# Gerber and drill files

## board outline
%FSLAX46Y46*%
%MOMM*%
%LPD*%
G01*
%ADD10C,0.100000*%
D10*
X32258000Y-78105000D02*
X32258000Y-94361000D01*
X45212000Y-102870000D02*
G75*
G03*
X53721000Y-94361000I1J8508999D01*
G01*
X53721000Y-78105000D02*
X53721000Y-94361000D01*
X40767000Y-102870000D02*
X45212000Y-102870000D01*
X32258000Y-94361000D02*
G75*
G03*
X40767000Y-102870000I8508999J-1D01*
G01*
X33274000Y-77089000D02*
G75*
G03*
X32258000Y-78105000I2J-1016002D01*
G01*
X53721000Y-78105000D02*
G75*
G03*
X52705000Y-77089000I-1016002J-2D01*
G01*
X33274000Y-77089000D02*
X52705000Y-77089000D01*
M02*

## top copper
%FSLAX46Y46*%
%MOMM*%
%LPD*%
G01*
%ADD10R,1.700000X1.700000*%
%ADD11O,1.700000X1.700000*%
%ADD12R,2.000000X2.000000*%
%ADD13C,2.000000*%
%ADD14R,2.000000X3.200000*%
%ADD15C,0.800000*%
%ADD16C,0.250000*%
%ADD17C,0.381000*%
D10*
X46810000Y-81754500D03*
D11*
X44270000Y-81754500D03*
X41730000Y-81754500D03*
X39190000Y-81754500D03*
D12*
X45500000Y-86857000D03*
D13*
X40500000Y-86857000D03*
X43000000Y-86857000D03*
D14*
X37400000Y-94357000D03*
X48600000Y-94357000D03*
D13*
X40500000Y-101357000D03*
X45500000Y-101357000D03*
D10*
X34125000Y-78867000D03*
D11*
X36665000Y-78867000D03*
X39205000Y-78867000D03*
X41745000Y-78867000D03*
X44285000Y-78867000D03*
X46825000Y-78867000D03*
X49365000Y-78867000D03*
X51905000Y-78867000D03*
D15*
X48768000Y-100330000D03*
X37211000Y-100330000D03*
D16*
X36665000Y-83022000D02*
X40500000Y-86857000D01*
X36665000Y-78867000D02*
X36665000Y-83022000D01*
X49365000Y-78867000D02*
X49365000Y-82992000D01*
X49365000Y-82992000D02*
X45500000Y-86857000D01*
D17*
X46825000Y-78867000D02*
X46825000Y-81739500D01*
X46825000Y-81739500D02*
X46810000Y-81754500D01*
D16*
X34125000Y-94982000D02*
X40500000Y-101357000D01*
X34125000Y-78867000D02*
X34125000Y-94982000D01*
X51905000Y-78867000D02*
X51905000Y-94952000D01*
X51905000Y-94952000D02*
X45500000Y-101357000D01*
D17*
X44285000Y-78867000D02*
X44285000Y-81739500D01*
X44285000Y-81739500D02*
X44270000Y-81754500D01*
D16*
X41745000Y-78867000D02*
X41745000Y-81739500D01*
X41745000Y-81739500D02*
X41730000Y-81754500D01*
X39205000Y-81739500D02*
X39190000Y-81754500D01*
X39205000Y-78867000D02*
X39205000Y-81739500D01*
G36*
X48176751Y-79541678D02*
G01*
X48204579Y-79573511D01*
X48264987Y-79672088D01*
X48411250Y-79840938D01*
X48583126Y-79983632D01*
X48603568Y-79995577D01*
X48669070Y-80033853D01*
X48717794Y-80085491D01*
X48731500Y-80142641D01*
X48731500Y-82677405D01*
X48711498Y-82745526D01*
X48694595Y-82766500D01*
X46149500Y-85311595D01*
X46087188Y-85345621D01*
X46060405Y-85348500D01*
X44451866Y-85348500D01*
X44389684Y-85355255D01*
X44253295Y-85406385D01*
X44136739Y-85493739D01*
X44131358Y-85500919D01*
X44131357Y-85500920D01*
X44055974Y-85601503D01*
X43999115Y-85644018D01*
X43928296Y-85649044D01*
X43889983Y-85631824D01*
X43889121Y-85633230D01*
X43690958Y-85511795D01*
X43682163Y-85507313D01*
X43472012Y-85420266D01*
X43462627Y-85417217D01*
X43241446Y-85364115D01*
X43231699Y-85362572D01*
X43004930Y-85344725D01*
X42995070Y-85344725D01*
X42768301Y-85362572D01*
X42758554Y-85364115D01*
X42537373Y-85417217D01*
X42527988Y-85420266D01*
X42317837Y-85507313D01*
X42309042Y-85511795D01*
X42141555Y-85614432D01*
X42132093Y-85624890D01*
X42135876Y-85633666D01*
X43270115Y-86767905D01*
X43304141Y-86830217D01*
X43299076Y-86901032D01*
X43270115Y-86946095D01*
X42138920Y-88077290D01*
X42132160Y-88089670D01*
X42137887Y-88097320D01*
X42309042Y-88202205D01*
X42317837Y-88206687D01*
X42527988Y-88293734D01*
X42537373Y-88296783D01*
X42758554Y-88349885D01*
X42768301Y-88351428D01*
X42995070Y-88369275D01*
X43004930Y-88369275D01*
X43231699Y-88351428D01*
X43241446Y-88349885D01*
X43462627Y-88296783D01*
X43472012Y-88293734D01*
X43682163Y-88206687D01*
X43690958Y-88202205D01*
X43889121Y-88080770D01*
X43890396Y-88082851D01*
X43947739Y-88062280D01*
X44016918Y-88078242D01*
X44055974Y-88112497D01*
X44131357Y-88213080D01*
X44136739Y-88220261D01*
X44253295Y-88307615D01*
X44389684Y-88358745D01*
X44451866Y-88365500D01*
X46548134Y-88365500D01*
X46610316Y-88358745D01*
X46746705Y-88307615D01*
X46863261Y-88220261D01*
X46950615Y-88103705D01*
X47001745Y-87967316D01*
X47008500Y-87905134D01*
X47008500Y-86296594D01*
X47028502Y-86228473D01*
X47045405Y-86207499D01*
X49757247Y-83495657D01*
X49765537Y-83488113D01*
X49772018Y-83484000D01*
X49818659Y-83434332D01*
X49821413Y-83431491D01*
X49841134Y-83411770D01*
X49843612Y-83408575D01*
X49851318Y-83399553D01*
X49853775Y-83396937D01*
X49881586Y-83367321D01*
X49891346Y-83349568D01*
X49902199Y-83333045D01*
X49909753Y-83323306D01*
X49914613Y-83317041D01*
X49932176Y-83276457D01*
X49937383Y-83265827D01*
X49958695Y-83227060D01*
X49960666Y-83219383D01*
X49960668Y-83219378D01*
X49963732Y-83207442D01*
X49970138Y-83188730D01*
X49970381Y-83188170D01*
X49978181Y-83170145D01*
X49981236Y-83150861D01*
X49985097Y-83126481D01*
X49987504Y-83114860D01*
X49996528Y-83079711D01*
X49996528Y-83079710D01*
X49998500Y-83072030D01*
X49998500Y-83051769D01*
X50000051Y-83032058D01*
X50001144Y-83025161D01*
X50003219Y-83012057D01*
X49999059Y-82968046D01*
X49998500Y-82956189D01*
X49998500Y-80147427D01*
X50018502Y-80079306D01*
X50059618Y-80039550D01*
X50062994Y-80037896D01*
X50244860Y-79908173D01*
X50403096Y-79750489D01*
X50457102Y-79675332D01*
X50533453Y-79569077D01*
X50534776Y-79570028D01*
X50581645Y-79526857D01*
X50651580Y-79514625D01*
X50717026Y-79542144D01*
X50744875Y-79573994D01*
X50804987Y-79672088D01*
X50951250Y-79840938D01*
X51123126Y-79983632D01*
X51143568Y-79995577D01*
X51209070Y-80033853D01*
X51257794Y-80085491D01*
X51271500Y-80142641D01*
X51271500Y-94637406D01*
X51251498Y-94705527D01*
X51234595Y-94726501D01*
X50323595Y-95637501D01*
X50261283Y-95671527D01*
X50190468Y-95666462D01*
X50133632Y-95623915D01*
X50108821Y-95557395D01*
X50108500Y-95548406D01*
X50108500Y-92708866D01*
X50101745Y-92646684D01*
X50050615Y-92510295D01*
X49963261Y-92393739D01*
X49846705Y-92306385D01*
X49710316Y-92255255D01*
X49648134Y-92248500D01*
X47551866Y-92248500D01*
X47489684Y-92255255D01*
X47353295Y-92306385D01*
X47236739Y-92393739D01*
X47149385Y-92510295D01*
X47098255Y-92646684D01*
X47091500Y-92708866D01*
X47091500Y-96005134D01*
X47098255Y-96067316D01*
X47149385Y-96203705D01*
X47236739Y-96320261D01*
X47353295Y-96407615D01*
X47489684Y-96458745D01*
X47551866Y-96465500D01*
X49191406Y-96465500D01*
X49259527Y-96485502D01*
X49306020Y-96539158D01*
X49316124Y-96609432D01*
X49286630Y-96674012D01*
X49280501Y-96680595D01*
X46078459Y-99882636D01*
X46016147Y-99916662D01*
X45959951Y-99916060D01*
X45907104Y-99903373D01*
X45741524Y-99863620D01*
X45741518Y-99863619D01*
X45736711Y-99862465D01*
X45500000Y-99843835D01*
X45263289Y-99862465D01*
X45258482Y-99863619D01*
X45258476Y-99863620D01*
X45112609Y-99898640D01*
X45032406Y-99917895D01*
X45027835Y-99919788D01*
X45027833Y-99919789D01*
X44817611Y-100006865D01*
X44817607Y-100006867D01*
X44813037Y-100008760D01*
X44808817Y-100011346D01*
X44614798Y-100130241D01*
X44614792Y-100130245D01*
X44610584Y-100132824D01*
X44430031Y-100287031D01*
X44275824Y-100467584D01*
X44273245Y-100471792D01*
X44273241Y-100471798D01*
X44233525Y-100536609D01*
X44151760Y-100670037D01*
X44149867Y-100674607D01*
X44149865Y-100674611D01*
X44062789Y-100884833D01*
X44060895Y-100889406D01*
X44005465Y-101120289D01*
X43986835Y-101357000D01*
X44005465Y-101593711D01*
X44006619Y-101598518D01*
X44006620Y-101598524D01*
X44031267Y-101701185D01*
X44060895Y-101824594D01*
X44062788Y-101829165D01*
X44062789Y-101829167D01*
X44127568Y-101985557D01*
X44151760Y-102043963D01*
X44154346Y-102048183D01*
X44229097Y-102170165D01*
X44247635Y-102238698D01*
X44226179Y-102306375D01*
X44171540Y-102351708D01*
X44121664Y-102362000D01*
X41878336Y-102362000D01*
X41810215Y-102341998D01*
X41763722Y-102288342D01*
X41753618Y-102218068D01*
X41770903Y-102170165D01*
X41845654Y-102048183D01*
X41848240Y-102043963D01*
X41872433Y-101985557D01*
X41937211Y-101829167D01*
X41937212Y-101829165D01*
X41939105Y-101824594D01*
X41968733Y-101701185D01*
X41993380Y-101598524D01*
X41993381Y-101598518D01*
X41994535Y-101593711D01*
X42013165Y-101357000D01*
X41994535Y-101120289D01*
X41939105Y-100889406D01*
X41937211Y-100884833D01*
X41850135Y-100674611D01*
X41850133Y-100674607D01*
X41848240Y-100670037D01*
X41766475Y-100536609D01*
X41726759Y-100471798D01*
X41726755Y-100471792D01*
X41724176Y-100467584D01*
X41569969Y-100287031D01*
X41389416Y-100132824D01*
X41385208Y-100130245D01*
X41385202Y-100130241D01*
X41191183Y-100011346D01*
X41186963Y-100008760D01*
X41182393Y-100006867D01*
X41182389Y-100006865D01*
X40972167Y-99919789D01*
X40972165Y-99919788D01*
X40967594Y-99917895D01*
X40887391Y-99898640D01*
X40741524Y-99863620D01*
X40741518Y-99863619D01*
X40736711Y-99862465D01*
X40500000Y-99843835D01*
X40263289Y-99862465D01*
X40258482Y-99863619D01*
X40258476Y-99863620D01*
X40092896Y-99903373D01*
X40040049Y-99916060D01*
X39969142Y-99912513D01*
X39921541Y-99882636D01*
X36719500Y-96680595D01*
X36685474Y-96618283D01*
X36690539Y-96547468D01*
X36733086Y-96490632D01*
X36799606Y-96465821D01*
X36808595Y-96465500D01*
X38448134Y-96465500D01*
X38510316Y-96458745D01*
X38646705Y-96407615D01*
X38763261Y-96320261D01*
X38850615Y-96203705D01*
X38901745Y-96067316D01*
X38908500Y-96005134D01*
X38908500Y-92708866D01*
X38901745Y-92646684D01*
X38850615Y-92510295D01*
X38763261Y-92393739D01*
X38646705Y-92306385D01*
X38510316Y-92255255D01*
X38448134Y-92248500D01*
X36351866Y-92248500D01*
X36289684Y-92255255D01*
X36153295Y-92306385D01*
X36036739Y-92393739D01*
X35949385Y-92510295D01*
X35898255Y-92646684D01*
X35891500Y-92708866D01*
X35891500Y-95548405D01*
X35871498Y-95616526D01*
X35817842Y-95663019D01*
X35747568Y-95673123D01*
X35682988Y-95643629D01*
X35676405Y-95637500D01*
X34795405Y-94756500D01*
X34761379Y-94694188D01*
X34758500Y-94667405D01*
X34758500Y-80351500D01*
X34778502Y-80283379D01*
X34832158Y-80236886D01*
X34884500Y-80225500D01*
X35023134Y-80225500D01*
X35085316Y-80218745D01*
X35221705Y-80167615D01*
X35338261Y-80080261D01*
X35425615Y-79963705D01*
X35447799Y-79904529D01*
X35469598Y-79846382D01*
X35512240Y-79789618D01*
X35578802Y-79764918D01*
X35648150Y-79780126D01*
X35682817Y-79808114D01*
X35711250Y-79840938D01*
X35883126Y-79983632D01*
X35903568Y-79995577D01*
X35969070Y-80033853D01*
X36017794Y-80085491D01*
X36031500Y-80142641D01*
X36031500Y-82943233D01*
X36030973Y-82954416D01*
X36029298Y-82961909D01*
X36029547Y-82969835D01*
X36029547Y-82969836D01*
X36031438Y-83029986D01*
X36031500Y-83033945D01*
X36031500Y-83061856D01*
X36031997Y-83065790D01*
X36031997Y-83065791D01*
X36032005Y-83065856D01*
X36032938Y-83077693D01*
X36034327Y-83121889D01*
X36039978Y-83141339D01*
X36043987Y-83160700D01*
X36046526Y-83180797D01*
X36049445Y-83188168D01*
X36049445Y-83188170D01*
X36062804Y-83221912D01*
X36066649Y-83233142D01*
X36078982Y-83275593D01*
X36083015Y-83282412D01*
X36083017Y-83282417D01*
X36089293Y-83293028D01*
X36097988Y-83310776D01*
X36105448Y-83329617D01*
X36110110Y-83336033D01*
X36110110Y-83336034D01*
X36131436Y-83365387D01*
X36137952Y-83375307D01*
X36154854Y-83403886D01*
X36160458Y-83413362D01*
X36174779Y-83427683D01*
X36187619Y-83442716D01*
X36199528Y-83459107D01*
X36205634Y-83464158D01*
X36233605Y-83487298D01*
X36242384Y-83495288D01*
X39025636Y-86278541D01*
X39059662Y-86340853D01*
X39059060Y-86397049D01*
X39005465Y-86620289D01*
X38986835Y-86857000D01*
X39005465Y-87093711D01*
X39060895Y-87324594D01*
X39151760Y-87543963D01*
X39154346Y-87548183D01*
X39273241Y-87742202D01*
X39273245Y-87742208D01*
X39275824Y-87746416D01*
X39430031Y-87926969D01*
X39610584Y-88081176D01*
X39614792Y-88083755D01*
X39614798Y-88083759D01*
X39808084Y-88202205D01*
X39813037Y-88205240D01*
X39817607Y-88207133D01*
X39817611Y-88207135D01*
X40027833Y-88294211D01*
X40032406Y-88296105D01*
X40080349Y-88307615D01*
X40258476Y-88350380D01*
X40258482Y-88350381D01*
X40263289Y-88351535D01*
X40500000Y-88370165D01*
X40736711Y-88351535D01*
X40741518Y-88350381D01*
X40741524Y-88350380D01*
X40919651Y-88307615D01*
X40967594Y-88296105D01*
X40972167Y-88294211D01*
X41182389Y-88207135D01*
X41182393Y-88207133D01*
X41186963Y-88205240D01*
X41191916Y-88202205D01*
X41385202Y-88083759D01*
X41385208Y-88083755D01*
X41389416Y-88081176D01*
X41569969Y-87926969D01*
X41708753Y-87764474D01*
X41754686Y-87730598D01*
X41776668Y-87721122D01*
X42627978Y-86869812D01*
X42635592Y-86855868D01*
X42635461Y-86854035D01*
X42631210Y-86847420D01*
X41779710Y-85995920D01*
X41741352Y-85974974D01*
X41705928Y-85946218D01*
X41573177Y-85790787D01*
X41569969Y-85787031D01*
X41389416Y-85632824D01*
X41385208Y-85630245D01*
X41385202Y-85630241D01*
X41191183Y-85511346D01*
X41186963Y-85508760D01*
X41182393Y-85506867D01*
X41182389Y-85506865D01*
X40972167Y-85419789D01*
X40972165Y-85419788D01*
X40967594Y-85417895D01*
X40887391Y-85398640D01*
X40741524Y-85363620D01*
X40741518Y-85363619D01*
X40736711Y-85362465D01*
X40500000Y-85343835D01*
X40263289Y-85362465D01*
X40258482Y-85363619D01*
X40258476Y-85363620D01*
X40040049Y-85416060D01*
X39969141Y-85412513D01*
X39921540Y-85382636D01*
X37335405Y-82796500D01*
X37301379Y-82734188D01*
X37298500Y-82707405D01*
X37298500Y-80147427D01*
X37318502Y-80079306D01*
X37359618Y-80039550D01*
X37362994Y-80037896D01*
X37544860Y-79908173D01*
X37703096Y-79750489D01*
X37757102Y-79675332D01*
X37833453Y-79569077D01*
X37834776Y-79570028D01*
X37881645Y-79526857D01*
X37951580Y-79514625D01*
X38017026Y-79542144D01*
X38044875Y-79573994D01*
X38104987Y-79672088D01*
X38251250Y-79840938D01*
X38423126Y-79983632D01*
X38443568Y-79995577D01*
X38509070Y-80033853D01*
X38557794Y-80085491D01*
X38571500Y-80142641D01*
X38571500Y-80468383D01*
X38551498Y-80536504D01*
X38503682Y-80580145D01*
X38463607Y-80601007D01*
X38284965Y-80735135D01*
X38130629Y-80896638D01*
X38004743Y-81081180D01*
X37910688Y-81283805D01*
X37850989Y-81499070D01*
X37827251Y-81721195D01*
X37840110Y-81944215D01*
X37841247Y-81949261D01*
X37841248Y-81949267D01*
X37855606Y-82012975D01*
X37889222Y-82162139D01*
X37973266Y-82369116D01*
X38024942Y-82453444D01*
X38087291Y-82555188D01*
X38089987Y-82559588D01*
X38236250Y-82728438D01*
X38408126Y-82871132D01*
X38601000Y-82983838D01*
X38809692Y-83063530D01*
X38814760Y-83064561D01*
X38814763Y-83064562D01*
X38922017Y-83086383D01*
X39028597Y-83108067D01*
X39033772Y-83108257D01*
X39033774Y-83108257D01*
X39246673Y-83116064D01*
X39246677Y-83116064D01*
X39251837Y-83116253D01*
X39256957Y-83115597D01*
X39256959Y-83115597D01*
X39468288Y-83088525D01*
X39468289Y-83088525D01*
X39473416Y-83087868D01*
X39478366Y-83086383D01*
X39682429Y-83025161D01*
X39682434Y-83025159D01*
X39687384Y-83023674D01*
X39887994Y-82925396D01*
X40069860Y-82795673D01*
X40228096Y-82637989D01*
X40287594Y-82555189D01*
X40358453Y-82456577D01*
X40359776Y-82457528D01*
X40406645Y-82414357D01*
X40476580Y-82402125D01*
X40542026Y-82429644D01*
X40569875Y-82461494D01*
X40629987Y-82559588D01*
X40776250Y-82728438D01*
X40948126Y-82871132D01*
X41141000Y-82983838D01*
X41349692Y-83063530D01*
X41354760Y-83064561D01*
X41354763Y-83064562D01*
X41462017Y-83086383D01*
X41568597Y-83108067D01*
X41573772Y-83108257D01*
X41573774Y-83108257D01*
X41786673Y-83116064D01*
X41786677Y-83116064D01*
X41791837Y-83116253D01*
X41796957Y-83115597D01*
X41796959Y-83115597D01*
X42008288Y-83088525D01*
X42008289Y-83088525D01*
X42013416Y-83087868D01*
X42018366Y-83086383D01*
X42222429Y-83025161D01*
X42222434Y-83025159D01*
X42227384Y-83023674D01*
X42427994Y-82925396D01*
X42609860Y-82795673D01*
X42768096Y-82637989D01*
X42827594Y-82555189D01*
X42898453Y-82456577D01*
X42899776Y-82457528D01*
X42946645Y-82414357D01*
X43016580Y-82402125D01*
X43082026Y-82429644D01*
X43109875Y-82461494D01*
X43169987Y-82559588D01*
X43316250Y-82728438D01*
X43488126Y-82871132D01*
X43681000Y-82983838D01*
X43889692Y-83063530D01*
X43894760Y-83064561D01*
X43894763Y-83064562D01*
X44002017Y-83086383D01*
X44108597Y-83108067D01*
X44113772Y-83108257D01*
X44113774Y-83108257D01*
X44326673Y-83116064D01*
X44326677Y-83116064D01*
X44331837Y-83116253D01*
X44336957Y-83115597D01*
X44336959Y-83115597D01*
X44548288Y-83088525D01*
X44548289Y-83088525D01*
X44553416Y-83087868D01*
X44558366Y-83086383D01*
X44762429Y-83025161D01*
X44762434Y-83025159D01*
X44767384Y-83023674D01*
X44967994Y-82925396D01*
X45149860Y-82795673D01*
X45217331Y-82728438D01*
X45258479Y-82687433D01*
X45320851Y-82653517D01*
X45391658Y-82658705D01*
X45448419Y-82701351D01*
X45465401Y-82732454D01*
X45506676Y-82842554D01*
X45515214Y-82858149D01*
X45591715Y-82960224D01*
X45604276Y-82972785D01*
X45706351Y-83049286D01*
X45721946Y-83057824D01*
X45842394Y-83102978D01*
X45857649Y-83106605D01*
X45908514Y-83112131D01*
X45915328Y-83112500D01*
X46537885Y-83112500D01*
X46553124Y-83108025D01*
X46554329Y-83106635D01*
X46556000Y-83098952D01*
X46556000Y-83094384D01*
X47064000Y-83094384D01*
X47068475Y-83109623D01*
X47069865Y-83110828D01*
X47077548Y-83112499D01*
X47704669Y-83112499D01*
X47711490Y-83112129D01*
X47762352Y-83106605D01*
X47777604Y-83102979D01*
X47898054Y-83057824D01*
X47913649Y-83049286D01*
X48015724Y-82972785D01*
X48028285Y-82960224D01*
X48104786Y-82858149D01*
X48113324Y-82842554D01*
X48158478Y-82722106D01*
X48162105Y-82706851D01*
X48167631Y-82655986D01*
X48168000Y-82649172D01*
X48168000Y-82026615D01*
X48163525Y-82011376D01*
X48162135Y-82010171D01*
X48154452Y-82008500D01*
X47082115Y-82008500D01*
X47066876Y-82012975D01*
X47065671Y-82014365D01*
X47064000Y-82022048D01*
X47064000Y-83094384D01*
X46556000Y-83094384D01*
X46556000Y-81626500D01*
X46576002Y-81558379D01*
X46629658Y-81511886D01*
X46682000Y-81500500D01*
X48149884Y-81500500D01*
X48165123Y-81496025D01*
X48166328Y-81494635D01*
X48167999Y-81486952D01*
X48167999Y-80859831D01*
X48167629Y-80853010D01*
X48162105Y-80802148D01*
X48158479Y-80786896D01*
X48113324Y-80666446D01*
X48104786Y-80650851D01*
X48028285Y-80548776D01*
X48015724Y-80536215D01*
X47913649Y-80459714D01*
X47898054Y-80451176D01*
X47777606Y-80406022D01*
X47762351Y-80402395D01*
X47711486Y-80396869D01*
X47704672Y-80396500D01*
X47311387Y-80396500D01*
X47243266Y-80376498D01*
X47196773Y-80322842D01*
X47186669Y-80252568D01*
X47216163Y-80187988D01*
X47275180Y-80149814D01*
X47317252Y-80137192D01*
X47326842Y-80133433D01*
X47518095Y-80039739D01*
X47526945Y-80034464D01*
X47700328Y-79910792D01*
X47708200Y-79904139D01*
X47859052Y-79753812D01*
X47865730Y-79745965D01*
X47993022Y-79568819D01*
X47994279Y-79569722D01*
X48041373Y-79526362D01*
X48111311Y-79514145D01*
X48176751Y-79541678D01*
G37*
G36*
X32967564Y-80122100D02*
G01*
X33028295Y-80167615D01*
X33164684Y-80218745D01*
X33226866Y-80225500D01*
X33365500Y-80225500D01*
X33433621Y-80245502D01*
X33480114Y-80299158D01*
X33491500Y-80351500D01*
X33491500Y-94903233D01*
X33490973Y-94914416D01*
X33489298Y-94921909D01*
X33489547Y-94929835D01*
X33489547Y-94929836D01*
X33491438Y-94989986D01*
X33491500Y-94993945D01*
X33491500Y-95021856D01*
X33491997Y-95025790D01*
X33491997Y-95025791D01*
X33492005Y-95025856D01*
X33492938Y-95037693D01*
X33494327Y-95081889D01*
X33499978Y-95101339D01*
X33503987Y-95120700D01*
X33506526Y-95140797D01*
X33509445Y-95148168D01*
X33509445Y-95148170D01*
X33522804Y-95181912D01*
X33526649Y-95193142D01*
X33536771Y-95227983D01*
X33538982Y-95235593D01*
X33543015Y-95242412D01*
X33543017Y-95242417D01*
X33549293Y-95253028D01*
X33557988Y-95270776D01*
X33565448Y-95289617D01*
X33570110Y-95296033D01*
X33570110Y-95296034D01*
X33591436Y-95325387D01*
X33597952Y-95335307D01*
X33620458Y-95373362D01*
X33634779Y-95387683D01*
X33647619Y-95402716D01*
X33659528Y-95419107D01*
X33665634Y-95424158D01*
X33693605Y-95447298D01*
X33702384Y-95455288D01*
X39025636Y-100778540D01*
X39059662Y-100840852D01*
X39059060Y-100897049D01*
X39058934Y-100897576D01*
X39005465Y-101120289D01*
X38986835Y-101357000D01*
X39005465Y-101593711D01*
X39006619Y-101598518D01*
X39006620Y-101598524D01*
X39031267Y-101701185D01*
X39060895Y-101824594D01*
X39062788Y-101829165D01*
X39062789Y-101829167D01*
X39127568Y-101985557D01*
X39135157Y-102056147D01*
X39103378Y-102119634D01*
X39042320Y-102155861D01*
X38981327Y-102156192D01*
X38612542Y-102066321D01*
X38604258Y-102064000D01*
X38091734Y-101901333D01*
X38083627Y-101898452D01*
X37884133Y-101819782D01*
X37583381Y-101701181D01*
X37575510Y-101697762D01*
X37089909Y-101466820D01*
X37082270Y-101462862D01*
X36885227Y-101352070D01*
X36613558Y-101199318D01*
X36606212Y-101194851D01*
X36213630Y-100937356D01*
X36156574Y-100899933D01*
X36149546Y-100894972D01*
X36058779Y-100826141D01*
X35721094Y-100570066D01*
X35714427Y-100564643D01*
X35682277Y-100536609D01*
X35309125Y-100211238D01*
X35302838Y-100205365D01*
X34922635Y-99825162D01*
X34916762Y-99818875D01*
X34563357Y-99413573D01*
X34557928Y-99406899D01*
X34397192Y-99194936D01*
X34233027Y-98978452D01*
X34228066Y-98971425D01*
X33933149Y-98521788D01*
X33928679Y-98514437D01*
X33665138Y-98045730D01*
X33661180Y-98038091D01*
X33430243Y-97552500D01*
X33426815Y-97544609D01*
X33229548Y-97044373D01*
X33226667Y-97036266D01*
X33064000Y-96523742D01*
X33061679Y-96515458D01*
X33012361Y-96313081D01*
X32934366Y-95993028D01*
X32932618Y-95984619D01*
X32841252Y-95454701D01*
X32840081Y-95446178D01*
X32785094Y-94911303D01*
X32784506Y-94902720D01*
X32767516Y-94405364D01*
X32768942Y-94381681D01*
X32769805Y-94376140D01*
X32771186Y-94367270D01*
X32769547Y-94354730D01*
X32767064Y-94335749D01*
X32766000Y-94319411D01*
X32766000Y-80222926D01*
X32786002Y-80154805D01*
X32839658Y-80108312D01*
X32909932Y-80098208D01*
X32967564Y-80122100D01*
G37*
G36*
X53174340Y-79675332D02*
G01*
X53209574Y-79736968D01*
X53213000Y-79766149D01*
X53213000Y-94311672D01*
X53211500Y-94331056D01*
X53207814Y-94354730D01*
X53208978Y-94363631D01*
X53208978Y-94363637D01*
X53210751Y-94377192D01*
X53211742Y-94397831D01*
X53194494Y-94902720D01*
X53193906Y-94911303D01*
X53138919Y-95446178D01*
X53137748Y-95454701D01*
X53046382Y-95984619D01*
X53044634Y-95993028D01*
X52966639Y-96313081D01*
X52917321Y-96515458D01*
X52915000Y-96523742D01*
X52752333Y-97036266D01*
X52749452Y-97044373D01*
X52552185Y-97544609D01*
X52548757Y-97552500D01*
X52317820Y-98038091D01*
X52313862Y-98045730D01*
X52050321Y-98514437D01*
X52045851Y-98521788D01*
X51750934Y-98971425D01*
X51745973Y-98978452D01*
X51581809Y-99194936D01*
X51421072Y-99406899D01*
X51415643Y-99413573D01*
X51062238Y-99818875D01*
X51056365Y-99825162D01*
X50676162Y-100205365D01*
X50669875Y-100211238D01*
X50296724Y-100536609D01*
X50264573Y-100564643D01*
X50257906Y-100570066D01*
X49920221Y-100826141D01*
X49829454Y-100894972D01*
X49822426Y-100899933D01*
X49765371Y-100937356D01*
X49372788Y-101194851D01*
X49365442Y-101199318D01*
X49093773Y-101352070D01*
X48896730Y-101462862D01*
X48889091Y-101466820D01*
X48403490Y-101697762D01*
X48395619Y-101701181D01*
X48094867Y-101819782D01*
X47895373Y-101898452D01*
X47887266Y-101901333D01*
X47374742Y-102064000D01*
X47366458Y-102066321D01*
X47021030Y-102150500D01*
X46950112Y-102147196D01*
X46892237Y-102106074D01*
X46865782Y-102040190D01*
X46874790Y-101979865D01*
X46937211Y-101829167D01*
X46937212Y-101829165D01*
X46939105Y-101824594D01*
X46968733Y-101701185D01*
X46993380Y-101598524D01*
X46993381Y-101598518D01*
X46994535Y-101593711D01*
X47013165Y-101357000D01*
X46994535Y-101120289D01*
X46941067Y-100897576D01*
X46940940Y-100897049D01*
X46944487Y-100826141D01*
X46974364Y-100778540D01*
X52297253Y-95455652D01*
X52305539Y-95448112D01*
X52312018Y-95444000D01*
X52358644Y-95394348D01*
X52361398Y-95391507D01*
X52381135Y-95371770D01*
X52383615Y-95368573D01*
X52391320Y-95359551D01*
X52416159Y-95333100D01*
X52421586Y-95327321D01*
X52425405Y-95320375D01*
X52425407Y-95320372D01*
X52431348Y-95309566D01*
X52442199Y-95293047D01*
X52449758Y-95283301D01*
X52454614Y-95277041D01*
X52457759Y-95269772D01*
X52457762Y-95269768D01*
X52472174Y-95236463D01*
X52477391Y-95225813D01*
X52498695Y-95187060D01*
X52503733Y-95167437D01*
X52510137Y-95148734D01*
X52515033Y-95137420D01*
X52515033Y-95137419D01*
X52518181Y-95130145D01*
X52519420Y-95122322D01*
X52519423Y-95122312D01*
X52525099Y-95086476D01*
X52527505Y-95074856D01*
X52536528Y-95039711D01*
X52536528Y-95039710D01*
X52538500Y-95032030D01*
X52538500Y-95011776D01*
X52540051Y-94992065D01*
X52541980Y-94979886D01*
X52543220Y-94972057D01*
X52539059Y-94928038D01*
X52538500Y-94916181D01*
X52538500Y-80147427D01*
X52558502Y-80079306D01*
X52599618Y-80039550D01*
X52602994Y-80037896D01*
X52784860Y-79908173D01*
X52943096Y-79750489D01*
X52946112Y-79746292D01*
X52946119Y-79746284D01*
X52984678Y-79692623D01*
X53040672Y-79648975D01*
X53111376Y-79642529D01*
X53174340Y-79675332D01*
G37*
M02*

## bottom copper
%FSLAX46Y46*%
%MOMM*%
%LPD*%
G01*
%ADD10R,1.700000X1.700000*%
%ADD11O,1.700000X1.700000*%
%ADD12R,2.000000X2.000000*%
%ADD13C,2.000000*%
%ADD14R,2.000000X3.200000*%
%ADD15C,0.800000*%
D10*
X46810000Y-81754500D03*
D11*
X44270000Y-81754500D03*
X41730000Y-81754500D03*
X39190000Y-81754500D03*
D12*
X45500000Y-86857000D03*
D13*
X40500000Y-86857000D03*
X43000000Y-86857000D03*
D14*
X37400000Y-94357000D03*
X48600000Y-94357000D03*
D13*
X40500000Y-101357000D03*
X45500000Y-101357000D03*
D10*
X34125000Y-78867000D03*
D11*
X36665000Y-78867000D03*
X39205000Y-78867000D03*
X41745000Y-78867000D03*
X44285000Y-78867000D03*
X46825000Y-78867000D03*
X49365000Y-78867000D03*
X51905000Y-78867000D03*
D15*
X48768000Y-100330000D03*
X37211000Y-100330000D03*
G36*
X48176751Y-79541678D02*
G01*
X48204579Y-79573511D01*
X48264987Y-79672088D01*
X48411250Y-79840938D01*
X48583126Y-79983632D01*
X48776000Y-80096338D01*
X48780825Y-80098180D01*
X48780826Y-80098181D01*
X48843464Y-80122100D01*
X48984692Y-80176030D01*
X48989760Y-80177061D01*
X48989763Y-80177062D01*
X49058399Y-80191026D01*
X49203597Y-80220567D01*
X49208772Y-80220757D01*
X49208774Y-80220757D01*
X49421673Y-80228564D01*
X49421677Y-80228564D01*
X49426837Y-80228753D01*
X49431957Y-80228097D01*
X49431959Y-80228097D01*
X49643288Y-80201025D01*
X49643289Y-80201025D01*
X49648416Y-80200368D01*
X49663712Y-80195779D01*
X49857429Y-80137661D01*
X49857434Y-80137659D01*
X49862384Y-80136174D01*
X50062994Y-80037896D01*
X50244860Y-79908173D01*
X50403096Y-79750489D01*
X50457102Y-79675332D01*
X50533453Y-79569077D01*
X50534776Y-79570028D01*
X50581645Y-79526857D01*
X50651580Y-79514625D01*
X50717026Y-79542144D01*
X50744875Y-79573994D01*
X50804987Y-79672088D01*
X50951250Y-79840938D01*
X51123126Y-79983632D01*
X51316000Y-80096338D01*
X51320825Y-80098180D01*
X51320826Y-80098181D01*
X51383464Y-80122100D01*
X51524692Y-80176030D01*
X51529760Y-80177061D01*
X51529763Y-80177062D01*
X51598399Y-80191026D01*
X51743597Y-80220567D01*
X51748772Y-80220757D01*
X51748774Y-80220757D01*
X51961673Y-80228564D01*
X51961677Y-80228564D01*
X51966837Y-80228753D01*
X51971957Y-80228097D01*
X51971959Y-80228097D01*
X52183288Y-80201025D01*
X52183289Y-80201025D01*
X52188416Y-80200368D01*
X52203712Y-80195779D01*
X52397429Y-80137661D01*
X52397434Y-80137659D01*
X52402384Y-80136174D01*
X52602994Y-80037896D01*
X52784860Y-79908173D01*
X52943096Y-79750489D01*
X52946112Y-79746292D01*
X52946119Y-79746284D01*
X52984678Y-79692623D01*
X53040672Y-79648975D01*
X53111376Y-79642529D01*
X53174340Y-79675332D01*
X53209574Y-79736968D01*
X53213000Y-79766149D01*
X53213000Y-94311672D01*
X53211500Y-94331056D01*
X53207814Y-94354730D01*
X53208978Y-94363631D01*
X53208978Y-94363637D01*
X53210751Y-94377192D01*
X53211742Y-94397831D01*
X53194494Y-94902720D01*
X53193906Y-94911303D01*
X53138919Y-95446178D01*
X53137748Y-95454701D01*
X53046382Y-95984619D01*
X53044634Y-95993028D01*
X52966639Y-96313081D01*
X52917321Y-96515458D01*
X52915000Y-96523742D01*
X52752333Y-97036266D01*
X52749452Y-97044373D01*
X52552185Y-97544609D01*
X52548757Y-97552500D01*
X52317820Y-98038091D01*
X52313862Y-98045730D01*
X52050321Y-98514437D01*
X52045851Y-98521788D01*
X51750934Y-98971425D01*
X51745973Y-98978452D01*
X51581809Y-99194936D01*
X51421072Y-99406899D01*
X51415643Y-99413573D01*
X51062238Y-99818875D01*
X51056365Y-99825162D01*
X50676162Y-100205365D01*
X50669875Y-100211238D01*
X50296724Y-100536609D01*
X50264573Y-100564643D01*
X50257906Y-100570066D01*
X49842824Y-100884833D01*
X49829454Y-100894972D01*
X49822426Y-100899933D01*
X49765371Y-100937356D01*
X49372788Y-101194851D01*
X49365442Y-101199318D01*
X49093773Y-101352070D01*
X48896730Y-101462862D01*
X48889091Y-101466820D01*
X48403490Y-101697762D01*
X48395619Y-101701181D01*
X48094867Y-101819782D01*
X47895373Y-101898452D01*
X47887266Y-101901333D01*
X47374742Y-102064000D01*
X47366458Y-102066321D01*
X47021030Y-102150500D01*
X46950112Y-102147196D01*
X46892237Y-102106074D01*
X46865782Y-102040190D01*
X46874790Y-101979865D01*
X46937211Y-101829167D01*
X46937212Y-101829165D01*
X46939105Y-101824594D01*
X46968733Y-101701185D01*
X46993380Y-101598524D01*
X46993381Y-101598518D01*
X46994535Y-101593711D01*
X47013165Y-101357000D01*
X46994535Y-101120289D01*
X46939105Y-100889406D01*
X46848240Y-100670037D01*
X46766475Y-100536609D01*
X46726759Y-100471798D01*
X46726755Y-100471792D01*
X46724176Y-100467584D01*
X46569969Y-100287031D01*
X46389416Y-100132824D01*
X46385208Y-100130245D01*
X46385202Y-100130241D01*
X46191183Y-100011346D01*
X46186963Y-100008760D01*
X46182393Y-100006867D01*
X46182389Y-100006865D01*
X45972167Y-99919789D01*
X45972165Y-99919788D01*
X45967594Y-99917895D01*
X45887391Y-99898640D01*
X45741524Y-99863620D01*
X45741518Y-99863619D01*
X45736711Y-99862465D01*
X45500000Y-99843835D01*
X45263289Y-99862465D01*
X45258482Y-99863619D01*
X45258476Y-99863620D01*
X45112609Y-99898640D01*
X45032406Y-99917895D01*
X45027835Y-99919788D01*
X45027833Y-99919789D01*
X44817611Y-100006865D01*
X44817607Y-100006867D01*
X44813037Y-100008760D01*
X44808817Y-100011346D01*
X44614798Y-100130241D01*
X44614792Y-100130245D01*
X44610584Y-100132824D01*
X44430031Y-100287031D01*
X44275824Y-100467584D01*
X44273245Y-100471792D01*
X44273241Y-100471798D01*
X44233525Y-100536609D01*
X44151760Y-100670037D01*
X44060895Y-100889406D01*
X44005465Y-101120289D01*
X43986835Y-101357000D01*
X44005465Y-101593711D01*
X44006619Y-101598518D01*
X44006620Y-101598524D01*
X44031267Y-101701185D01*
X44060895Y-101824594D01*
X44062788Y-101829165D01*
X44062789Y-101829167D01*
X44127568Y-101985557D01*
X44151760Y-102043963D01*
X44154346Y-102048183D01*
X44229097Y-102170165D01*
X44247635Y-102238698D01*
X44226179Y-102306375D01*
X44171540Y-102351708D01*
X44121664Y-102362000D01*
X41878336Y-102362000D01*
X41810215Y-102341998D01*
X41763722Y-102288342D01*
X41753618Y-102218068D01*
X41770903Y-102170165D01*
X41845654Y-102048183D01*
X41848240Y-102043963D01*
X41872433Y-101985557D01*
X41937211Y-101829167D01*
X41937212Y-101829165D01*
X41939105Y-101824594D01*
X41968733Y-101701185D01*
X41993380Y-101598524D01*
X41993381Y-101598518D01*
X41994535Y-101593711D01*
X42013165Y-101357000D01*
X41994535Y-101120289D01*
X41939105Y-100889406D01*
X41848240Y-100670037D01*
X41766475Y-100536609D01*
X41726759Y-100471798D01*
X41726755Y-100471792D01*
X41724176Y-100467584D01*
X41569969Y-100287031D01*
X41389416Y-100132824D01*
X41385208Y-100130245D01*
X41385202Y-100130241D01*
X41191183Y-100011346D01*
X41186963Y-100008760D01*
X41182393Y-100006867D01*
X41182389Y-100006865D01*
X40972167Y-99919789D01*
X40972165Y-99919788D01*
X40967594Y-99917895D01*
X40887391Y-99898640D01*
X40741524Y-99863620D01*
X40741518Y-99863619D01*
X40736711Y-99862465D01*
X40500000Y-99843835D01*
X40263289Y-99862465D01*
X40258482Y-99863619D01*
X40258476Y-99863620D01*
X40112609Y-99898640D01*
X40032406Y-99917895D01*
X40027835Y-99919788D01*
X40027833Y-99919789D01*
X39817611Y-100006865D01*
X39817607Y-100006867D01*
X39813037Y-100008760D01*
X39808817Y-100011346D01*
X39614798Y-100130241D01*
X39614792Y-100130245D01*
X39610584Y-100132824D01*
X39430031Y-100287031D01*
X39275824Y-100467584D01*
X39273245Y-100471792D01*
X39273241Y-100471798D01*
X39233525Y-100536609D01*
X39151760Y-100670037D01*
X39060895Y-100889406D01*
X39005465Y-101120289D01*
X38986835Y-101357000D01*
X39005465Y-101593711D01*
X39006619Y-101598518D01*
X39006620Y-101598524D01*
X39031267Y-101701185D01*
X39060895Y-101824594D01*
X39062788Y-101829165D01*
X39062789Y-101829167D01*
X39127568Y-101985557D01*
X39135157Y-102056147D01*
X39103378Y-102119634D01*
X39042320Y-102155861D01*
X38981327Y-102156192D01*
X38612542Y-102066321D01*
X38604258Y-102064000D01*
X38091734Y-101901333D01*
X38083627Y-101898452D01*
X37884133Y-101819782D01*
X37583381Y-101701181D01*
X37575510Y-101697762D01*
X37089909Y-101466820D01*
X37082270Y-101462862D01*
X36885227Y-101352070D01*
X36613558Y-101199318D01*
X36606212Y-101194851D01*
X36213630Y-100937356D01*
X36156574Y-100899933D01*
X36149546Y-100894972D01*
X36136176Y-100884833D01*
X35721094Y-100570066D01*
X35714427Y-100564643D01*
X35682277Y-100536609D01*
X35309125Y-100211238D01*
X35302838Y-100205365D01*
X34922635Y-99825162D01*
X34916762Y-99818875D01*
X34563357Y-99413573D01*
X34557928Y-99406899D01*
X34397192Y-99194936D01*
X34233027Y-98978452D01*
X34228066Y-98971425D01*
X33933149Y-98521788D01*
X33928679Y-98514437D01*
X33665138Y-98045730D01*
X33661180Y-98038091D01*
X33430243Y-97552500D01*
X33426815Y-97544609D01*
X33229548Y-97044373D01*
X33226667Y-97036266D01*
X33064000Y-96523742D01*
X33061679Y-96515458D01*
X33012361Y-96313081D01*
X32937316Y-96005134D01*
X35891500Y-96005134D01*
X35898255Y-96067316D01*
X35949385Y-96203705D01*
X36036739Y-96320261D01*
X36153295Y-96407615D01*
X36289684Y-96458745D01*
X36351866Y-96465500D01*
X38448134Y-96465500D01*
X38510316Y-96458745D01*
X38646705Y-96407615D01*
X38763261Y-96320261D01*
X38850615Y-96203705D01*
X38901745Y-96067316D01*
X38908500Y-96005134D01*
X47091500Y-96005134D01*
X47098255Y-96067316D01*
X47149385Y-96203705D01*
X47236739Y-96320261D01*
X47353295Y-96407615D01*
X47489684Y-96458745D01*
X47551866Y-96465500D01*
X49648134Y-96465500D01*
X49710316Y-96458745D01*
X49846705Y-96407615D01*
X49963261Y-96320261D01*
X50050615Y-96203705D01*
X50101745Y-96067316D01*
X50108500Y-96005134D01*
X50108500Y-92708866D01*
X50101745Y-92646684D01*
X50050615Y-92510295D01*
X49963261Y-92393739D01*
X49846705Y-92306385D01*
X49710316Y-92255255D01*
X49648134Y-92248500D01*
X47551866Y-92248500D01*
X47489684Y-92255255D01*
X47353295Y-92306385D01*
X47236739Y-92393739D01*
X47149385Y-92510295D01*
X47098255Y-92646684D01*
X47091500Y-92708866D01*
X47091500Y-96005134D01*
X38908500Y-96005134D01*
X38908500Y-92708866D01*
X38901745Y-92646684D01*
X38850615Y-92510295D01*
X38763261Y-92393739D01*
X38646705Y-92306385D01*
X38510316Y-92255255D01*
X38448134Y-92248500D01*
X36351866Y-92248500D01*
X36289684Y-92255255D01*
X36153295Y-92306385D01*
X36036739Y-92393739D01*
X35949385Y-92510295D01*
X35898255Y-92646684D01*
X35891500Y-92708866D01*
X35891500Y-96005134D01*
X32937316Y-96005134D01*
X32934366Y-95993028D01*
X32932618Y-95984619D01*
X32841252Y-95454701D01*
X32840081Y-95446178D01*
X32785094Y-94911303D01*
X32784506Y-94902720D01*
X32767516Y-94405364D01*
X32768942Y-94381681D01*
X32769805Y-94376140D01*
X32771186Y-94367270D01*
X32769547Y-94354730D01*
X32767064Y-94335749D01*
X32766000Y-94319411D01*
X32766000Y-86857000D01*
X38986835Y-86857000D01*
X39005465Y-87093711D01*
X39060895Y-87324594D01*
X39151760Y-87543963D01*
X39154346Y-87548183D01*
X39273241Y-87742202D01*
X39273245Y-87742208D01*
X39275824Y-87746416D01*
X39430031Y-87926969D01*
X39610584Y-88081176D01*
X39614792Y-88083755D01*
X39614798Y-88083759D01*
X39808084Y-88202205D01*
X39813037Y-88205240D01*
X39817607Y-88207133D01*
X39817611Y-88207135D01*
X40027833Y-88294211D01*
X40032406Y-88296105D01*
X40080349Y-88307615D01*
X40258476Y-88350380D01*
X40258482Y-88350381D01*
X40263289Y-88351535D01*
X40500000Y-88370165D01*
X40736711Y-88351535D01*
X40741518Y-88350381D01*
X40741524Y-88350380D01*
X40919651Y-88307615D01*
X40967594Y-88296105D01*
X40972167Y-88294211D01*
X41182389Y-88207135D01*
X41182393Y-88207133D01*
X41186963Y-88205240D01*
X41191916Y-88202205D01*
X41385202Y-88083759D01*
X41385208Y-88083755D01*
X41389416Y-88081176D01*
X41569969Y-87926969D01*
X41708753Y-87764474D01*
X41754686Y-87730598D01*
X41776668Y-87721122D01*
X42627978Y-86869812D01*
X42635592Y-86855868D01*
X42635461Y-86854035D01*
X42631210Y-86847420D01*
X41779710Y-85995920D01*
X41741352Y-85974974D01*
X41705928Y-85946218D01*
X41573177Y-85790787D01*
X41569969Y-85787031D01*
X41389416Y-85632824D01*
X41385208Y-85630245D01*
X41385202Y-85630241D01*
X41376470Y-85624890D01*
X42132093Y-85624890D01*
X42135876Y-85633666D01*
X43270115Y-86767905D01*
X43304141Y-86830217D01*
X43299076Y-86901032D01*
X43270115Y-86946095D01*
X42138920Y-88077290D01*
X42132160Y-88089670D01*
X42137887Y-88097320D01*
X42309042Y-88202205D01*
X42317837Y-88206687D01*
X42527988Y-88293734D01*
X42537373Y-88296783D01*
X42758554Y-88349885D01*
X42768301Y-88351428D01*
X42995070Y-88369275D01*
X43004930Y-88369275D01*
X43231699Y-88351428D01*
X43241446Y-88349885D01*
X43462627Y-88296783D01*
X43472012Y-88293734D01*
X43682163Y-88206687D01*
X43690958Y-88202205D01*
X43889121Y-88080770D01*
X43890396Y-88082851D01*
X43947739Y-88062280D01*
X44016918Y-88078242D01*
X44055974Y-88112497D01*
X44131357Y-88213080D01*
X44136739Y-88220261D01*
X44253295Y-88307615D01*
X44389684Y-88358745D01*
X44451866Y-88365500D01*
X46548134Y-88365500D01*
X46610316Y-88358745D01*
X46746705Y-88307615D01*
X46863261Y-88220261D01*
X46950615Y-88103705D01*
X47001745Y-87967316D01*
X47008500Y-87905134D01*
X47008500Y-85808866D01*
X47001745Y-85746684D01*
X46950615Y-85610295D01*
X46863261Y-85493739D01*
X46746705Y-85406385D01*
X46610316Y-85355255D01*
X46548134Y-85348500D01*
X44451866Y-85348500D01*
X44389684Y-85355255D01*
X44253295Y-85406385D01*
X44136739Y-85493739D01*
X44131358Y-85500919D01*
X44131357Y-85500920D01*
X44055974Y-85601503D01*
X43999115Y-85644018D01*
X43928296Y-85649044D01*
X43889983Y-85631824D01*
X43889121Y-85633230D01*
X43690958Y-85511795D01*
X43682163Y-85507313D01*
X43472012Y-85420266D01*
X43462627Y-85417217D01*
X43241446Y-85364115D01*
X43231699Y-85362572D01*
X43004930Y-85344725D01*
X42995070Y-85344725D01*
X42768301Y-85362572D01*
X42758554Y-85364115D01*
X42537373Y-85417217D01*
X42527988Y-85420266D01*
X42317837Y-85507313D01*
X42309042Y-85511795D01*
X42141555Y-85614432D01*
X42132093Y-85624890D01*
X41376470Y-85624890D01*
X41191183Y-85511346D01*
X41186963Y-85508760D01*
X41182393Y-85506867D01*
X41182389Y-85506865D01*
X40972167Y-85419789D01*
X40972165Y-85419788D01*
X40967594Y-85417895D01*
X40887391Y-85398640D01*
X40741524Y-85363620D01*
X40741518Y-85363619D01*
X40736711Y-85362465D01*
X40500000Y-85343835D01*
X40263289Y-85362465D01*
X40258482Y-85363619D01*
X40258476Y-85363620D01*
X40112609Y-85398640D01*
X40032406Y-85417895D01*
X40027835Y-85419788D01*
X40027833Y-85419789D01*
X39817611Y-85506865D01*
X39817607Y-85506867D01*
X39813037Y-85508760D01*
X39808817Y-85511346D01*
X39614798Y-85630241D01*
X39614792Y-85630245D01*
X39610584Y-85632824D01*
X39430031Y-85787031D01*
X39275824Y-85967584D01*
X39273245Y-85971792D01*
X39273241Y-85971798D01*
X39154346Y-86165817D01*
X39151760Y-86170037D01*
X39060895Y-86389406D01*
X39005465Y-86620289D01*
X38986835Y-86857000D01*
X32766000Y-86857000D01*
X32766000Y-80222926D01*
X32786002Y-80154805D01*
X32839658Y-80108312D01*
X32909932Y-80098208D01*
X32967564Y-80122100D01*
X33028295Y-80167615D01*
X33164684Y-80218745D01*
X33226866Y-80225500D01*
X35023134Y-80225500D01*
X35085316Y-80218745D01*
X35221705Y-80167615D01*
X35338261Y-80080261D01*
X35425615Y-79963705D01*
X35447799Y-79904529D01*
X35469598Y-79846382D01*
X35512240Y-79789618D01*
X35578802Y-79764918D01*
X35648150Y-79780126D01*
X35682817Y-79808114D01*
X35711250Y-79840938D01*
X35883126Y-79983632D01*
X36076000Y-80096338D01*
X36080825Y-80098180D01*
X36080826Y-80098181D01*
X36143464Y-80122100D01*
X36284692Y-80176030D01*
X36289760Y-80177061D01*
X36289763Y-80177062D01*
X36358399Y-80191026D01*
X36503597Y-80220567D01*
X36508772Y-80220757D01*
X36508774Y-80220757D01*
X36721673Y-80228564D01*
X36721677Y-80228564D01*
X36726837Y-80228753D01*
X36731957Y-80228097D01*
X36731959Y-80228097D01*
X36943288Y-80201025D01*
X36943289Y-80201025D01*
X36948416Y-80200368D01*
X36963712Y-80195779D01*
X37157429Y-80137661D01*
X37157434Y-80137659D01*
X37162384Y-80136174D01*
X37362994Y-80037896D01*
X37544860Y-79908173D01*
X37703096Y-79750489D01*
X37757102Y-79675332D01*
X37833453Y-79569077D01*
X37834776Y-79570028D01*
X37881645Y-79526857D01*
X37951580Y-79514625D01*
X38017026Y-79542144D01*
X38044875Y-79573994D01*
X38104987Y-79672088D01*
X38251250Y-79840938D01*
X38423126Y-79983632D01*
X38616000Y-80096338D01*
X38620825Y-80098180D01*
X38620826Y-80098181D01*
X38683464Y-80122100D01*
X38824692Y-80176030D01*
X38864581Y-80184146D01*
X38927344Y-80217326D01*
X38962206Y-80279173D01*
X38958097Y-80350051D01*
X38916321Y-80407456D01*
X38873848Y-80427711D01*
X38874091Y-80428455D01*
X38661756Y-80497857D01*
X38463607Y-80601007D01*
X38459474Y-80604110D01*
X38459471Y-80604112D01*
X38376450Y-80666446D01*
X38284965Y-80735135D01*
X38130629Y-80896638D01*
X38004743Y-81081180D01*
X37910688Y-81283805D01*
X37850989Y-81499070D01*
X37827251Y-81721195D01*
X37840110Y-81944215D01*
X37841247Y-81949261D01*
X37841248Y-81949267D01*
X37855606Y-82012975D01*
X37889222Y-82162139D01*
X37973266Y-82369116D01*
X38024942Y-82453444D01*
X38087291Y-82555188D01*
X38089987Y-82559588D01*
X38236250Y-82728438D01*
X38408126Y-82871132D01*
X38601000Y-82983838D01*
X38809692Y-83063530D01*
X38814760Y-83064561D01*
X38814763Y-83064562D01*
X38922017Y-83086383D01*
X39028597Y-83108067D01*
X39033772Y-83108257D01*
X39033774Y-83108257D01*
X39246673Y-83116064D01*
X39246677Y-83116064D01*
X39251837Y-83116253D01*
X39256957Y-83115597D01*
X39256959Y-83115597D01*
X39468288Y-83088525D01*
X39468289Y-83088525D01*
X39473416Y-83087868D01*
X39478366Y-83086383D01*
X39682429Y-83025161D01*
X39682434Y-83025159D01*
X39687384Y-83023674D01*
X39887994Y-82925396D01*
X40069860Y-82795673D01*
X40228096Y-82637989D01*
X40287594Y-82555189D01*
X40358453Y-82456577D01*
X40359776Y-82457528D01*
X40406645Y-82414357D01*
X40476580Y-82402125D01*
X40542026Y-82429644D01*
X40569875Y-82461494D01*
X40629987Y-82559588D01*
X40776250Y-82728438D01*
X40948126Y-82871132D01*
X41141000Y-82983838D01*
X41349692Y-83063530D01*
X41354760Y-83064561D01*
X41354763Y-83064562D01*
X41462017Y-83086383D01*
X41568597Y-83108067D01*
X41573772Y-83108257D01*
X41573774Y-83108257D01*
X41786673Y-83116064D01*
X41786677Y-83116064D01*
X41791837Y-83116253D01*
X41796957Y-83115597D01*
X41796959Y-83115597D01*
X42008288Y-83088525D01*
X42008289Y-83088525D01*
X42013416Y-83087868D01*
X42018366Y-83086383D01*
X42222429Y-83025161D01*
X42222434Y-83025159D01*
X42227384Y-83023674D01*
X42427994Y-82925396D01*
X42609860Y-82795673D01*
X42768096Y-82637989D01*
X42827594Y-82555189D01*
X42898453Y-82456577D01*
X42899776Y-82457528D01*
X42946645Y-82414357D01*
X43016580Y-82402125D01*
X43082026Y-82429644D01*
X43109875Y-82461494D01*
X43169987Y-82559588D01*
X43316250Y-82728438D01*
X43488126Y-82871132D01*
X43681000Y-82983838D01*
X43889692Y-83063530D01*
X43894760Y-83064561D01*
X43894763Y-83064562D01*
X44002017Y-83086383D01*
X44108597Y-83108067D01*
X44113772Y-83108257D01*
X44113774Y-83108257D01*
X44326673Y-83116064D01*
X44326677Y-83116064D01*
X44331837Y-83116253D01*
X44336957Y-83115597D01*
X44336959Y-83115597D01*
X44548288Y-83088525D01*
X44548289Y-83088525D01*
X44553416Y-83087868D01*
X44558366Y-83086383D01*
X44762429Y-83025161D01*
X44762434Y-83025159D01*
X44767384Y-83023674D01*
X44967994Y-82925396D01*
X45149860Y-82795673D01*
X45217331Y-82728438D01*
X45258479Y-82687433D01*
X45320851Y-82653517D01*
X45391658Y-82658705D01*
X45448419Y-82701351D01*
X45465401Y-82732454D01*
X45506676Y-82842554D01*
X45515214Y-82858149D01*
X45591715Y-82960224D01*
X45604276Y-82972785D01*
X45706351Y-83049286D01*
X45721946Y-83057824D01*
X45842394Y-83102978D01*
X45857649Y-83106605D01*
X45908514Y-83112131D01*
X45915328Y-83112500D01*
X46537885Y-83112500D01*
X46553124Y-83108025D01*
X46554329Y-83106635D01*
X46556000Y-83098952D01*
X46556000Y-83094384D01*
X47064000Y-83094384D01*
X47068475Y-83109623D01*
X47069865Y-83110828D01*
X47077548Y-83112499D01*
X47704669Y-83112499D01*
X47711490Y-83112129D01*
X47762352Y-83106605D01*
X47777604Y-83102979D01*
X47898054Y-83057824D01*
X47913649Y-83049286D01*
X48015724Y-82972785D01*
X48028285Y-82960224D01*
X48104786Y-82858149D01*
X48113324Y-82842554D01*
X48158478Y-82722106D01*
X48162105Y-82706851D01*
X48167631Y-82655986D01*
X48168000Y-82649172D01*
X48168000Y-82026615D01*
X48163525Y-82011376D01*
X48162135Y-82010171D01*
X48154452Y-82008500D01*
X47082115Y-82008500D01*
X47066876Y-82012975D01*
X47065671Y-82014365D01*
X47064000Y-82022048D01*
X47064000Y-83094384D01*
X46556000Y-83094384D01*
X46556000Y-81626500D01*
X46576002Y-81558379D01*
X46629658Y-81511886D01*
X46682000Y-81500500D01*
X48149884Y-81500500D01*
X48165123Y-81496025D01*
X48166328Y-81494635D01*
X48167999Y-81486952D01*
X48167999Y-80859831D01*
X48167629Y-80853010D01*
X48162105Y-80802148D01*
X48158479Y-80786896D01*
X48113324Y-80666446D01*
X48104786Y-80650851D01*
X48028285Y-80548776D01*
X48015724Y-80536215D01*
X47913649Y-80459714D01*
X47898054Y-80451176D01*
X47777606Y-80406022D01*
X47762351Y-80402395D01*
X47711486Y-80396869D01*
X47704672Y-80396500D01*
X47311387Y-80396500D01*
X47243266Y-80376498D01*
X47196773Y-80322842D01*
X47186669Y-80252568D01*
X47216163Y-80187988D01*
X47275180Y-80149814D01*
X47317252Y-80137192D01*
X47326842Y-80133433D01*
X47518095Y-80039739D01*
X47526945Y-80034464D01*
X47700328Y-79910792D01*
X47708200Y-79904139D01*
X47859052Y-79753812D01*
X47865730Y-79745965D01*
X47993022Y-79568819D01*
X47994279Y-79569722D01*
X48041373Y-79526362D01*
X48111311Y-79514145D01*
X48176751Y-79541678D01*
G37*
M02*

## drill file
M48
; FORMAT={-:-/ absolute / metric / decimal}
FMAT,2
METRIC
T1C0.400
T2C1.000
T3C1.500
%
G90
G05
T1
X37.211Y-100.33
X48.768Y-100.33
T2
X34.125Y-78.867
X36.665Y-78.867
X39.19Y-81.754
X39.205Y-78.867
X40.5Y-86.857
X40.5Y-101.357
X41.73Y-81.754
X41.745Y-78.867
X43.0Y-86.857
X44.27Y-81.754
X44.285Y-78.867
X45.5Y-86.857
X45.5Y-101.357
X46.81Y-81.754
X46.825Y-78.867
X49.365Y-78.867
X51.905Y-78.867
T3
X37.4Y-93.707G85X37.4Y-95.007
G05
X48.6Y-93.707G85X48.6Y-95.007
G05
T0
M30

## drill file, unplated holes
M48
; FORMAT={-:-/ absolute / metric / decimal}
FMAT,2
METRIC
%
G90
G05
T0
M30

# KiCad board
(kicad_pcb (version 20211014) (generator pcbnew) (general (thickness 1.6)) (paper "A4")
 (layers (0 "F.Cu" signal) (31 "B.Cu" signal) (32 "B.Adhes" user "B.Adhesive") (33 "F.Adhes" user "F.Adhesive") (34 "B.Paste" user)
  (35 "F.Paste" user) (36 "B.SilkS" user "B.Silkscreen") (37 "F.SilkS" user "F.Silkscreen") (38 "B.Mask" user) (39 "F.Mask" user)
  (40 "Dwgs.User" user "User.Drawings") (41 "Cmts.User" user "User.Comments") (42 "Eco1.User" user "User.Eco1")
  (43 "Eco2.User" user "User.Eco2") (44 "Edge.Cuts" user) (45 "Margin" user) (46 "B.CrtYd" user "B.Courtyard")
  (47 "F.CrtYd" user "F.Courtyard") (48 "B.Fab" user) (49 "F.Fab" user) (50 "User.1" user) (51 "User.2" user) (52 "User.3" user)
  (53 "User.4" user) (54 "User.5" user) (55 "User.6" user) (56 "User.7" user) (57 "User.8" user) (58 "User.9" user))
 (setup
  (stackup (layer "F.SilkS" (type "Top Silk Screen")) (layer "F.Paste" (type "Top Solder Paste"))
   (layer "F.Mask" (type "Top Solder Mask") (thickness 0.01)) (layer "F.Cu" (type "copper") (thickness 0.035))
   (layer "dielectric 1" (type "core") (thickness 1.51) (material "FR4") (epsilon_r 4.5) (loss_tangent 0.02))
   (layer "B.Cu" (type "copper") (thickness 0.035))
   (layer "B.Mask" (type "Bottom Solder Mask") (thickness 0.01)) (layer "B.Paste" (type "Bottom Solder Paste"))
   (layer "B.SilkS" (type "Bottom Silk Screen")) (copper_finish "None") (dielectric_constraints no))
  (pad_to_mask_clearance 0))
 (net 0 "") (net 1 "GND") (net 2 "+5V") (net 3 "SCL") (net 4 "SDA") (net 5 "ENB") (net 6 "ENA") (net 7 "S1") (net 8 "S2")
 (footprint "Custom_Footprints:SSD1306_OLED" (layer "F.Cu") (at 43 64 90)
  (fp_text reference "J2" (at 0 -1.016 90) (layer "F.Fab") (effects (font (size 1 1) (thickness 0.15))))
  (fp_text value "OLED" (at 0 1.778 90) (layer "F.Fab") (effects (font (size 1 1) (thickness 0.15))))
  (pad "1" thru_hole rect (at -17.7545 3.81 90) (size 1.7 1.7) (drill 1) (layers *.Cu *.Mask) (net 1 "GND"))
  (pad "2" thru_hole oval (at -17.7545 1.27 90) (size 1.7 1.7) (drill 1) (layers *.Cu *.Mask) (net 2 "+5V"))
  (pad "3" thru_hole oval (at -17.7545 -1.27 90) (size 1.7 1.7) (drill 1) (layers *.Cu *.Mask) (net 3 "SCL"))
  (pad "4" thru_hole oval (at -17.7545 -3.81 90) (size 1.7 1.7) (drill 1) (layers *.Cu *.Mask) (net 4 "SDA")))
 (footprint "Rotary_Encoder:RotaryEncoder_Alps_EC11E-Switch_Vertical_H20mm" (layer "F.Cu") (at 45.5 86.857 -90)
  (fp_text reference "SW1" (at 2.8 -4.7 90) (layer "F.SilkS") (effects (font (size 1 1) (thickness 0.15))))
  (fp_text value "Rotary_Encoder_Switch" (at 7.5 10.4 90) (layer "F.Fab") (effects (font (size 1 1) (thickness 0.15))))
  (pad "A" thru_hole rect (at 0 0 270) (size 2 2) (drill 1) (layers *.Cu *.Mask) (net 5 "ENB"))
  (pad "B" thru_hole circle (at 0 5 270) (size 2 2) (drill 1) (layers *.Cu *.Mask) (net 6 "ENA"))
  (pad "C" thru_hole circle (at 0 2.5 270) (size 2 2) (drill 1) (layers *.Cu *.Mask) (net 1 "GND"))
  (pad "MP" thru_hole rect (at 7.5 8.1 270) (size 3.2 2) (drill oval 2.8 1.5) (layers *.Cu *.Mask))
  (pad "MP" thru_hole rect (at 7.5 -3.1 270) (size 3.2 2) (drill oval 2.8 1.5) (layers *.Cu *.Mask))
  (pad "S1" thru_hole circle (at 14.5 5 270) (size 2 2) (drill 1) (layers *.Cu *.Mask) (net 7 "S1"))
  (pad "S2" thru_hole circle (at 14.5 0 270) (size 2 2) (drill 1) (layers *.Cu *.Mask) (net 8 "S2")))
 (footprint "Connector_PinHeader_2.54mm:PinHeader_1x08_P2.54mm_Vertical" (layer "F.Cu") (at 34.125 78.867 90)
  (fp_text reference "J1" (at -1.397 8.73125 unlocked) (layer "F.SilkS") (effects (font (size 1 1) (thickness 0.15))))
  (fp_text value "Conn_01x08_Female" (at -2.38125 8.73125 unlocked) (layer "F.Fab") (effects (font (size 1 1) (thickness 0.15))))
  (pad "1" thru_hole rect (at 0 0 90) (size 1.7 1.7) (drill 1) (layers *.Cu *.Mask) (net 7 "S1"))
  (pad "2" thru_hole oval (at 0 2.54 90) (size 1.7 1.7) (drill 1) (layers *.Cu *.Mask) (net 6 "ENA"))
  (pad "3" thru_hole oval (at 0 5.08 90) (size 1.7 1.7) (drill 1) (layers *.Cu *.Mask) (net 4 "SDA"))
  (pad "4" thru_hole oval (at 0 7.62 90) (size 1.7 1.7) (drill 1) (layers *.Cu *.Mask) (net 3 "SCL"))
  (pad "5" thru_hole oval (at 0 10.16 90) (size 1.7 1.7) (drill 1) (layers *.Cu *.Mask) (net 2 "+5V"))
  (pad "6" thru_hole oval (at 0 12.7 90) (size 1.7 1.7) (drill 1) (layers *.Cu *.Mask) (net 1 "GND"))
  (pad "7" thru_hole oval (at 0 15.24 90) (size 1.7 1.7) (drill 1) (layers *.Cu *.Mask) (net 5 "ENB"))
  (pad "8" thru_hole oval (at 0 17.78 90) (size 1.7 1.7) (drill 1) (layers *.Cu *.Mask) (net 8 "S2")))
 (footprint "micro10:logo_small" (layer "B.Cu") (at 42.926 94.361 90)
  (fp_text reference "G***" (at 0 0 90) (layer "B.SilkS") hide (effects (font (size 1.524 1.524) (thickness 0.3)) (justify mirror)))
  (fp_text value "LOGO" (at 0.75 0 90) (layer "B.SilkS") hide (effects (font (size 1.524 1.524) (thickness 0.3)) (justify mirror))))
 (gr_line (start 32.258 78.105) (end 32.258 94.361) (layer "Edge.Cuts") (width 0.1))
 (gr_arc (start 53.721 94.361) (mid 51.228772 100.377772) (end 45.212 102.87) (layer "Edge.Cuts") (width 0.1))
 (gr_line (start 53.721 78.105) (end 53.721 94.361) (layer "Edge.Cuts") (width 0.1))
 (gr_line (start 40.767 102.87) (end 45.212 102.87) (layer "Edge.Cuts") (width 0.1))
 (gr_arc (start 40.767 102.87) (mid 34.750228 100.377772) (end 32.258 94.361) (layer "Edge.Cuts") (width 0.1))
 (gr_arc (start 32.258 78.105) (mid 32.55558 77.38658) (end 33.274 77.089) (layer "Edge.Cuts") (width 0.1))
 (gr_arc (start 52.705 77.089) (mid 53.42342 77.38658) (end 53.721 78.105) (layer "Edge.Cuts") (width 0.1))
 (gr_line (start 33.274 77.089) (end 52.705 77.089) (layer "Edge.Cuts") (width 0.1))
 (segment (start 36.665 83.022) (end 40.5 86.857) (width 0.25) (layer "F.Cu") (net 6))
 (segment (start 36.665 78.867) (end 36.665 83.022) (width 0.25) (layer "F.Cu") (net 6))
 (segment (start 49.365 78.867) (end 49.365 82.992) (width 0.25) (layer "F.Cu") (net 5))
 (segment (start 49.365 82.992) (end 45.5 86.857) (width 0.25) (layer "F.Cu") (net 5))
 (segment (start 46.825 78.867) (end 46.825 81.7395) (width 0.381) (layer "F.Cu") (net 1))
 (segment (start 46.825 81.7395) (end 46.81 81.7545) (width 0.381) (layer "F.Cu") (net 1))
 (via (at 48.768 100.33) (size 0.8) (drill 0.4) (layers "F.Cu" "B.Cu") (free) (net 1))
 (via (at 37.211 100.33) (size 0.8) (drill 0.4) (layers "F.Cu" "B.Cu") (free) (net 1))
 (segment (start 34.125 94.982) (end 40.5 101.357) (width 0.25) (layer "F.Cu") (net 7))
 (segment (start 34.125 78.867) (end 34.125 94.982) (width 0.25) (layer "F.Cu") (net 7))
 (segment (start 51.905 78.867) (end 51.905 94.952) (width 0.25) (layer "F.Cu") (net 8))
 (segment (start 51.905 94.952) (end 45.5 101.357) (width 0.25) (layer "F.Cu") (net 8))
 (segment (start 44.285 78.867) (end 44.285 81.7395) (width 0.381) (layer "F.Cu") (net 2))
 (segment (start 44.285 81.7395) (end 44.27 81.7545) (width 0.381) (layer "F.Cu") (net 2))
 (segment (start 41.745 78.867) (end 41.745 81.7395) (width 0.25) (layer "F.Cu") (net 3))
 (segment (start 41.745 81.7395) (end 41.73 81.7545) (width 0.25) (layer "F.Cu") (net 3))
 (segment (start 39.205 81.7395) (end 39.19 81.7545) (width 0.25) (layer "F.Cu") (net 4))
 (segment (start 39.205 78.867) (end 39.205 81.7395) (width 0.25) (layer "F.Cu") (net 4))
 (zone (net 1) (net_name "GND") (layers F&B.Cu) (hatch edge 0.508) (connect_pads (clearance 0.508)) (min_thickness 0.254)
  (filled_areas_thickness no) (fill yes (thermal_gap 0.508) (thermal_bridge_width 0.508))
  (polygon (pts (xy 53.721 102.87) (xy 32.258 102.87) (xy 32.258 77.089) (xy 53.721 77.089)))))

